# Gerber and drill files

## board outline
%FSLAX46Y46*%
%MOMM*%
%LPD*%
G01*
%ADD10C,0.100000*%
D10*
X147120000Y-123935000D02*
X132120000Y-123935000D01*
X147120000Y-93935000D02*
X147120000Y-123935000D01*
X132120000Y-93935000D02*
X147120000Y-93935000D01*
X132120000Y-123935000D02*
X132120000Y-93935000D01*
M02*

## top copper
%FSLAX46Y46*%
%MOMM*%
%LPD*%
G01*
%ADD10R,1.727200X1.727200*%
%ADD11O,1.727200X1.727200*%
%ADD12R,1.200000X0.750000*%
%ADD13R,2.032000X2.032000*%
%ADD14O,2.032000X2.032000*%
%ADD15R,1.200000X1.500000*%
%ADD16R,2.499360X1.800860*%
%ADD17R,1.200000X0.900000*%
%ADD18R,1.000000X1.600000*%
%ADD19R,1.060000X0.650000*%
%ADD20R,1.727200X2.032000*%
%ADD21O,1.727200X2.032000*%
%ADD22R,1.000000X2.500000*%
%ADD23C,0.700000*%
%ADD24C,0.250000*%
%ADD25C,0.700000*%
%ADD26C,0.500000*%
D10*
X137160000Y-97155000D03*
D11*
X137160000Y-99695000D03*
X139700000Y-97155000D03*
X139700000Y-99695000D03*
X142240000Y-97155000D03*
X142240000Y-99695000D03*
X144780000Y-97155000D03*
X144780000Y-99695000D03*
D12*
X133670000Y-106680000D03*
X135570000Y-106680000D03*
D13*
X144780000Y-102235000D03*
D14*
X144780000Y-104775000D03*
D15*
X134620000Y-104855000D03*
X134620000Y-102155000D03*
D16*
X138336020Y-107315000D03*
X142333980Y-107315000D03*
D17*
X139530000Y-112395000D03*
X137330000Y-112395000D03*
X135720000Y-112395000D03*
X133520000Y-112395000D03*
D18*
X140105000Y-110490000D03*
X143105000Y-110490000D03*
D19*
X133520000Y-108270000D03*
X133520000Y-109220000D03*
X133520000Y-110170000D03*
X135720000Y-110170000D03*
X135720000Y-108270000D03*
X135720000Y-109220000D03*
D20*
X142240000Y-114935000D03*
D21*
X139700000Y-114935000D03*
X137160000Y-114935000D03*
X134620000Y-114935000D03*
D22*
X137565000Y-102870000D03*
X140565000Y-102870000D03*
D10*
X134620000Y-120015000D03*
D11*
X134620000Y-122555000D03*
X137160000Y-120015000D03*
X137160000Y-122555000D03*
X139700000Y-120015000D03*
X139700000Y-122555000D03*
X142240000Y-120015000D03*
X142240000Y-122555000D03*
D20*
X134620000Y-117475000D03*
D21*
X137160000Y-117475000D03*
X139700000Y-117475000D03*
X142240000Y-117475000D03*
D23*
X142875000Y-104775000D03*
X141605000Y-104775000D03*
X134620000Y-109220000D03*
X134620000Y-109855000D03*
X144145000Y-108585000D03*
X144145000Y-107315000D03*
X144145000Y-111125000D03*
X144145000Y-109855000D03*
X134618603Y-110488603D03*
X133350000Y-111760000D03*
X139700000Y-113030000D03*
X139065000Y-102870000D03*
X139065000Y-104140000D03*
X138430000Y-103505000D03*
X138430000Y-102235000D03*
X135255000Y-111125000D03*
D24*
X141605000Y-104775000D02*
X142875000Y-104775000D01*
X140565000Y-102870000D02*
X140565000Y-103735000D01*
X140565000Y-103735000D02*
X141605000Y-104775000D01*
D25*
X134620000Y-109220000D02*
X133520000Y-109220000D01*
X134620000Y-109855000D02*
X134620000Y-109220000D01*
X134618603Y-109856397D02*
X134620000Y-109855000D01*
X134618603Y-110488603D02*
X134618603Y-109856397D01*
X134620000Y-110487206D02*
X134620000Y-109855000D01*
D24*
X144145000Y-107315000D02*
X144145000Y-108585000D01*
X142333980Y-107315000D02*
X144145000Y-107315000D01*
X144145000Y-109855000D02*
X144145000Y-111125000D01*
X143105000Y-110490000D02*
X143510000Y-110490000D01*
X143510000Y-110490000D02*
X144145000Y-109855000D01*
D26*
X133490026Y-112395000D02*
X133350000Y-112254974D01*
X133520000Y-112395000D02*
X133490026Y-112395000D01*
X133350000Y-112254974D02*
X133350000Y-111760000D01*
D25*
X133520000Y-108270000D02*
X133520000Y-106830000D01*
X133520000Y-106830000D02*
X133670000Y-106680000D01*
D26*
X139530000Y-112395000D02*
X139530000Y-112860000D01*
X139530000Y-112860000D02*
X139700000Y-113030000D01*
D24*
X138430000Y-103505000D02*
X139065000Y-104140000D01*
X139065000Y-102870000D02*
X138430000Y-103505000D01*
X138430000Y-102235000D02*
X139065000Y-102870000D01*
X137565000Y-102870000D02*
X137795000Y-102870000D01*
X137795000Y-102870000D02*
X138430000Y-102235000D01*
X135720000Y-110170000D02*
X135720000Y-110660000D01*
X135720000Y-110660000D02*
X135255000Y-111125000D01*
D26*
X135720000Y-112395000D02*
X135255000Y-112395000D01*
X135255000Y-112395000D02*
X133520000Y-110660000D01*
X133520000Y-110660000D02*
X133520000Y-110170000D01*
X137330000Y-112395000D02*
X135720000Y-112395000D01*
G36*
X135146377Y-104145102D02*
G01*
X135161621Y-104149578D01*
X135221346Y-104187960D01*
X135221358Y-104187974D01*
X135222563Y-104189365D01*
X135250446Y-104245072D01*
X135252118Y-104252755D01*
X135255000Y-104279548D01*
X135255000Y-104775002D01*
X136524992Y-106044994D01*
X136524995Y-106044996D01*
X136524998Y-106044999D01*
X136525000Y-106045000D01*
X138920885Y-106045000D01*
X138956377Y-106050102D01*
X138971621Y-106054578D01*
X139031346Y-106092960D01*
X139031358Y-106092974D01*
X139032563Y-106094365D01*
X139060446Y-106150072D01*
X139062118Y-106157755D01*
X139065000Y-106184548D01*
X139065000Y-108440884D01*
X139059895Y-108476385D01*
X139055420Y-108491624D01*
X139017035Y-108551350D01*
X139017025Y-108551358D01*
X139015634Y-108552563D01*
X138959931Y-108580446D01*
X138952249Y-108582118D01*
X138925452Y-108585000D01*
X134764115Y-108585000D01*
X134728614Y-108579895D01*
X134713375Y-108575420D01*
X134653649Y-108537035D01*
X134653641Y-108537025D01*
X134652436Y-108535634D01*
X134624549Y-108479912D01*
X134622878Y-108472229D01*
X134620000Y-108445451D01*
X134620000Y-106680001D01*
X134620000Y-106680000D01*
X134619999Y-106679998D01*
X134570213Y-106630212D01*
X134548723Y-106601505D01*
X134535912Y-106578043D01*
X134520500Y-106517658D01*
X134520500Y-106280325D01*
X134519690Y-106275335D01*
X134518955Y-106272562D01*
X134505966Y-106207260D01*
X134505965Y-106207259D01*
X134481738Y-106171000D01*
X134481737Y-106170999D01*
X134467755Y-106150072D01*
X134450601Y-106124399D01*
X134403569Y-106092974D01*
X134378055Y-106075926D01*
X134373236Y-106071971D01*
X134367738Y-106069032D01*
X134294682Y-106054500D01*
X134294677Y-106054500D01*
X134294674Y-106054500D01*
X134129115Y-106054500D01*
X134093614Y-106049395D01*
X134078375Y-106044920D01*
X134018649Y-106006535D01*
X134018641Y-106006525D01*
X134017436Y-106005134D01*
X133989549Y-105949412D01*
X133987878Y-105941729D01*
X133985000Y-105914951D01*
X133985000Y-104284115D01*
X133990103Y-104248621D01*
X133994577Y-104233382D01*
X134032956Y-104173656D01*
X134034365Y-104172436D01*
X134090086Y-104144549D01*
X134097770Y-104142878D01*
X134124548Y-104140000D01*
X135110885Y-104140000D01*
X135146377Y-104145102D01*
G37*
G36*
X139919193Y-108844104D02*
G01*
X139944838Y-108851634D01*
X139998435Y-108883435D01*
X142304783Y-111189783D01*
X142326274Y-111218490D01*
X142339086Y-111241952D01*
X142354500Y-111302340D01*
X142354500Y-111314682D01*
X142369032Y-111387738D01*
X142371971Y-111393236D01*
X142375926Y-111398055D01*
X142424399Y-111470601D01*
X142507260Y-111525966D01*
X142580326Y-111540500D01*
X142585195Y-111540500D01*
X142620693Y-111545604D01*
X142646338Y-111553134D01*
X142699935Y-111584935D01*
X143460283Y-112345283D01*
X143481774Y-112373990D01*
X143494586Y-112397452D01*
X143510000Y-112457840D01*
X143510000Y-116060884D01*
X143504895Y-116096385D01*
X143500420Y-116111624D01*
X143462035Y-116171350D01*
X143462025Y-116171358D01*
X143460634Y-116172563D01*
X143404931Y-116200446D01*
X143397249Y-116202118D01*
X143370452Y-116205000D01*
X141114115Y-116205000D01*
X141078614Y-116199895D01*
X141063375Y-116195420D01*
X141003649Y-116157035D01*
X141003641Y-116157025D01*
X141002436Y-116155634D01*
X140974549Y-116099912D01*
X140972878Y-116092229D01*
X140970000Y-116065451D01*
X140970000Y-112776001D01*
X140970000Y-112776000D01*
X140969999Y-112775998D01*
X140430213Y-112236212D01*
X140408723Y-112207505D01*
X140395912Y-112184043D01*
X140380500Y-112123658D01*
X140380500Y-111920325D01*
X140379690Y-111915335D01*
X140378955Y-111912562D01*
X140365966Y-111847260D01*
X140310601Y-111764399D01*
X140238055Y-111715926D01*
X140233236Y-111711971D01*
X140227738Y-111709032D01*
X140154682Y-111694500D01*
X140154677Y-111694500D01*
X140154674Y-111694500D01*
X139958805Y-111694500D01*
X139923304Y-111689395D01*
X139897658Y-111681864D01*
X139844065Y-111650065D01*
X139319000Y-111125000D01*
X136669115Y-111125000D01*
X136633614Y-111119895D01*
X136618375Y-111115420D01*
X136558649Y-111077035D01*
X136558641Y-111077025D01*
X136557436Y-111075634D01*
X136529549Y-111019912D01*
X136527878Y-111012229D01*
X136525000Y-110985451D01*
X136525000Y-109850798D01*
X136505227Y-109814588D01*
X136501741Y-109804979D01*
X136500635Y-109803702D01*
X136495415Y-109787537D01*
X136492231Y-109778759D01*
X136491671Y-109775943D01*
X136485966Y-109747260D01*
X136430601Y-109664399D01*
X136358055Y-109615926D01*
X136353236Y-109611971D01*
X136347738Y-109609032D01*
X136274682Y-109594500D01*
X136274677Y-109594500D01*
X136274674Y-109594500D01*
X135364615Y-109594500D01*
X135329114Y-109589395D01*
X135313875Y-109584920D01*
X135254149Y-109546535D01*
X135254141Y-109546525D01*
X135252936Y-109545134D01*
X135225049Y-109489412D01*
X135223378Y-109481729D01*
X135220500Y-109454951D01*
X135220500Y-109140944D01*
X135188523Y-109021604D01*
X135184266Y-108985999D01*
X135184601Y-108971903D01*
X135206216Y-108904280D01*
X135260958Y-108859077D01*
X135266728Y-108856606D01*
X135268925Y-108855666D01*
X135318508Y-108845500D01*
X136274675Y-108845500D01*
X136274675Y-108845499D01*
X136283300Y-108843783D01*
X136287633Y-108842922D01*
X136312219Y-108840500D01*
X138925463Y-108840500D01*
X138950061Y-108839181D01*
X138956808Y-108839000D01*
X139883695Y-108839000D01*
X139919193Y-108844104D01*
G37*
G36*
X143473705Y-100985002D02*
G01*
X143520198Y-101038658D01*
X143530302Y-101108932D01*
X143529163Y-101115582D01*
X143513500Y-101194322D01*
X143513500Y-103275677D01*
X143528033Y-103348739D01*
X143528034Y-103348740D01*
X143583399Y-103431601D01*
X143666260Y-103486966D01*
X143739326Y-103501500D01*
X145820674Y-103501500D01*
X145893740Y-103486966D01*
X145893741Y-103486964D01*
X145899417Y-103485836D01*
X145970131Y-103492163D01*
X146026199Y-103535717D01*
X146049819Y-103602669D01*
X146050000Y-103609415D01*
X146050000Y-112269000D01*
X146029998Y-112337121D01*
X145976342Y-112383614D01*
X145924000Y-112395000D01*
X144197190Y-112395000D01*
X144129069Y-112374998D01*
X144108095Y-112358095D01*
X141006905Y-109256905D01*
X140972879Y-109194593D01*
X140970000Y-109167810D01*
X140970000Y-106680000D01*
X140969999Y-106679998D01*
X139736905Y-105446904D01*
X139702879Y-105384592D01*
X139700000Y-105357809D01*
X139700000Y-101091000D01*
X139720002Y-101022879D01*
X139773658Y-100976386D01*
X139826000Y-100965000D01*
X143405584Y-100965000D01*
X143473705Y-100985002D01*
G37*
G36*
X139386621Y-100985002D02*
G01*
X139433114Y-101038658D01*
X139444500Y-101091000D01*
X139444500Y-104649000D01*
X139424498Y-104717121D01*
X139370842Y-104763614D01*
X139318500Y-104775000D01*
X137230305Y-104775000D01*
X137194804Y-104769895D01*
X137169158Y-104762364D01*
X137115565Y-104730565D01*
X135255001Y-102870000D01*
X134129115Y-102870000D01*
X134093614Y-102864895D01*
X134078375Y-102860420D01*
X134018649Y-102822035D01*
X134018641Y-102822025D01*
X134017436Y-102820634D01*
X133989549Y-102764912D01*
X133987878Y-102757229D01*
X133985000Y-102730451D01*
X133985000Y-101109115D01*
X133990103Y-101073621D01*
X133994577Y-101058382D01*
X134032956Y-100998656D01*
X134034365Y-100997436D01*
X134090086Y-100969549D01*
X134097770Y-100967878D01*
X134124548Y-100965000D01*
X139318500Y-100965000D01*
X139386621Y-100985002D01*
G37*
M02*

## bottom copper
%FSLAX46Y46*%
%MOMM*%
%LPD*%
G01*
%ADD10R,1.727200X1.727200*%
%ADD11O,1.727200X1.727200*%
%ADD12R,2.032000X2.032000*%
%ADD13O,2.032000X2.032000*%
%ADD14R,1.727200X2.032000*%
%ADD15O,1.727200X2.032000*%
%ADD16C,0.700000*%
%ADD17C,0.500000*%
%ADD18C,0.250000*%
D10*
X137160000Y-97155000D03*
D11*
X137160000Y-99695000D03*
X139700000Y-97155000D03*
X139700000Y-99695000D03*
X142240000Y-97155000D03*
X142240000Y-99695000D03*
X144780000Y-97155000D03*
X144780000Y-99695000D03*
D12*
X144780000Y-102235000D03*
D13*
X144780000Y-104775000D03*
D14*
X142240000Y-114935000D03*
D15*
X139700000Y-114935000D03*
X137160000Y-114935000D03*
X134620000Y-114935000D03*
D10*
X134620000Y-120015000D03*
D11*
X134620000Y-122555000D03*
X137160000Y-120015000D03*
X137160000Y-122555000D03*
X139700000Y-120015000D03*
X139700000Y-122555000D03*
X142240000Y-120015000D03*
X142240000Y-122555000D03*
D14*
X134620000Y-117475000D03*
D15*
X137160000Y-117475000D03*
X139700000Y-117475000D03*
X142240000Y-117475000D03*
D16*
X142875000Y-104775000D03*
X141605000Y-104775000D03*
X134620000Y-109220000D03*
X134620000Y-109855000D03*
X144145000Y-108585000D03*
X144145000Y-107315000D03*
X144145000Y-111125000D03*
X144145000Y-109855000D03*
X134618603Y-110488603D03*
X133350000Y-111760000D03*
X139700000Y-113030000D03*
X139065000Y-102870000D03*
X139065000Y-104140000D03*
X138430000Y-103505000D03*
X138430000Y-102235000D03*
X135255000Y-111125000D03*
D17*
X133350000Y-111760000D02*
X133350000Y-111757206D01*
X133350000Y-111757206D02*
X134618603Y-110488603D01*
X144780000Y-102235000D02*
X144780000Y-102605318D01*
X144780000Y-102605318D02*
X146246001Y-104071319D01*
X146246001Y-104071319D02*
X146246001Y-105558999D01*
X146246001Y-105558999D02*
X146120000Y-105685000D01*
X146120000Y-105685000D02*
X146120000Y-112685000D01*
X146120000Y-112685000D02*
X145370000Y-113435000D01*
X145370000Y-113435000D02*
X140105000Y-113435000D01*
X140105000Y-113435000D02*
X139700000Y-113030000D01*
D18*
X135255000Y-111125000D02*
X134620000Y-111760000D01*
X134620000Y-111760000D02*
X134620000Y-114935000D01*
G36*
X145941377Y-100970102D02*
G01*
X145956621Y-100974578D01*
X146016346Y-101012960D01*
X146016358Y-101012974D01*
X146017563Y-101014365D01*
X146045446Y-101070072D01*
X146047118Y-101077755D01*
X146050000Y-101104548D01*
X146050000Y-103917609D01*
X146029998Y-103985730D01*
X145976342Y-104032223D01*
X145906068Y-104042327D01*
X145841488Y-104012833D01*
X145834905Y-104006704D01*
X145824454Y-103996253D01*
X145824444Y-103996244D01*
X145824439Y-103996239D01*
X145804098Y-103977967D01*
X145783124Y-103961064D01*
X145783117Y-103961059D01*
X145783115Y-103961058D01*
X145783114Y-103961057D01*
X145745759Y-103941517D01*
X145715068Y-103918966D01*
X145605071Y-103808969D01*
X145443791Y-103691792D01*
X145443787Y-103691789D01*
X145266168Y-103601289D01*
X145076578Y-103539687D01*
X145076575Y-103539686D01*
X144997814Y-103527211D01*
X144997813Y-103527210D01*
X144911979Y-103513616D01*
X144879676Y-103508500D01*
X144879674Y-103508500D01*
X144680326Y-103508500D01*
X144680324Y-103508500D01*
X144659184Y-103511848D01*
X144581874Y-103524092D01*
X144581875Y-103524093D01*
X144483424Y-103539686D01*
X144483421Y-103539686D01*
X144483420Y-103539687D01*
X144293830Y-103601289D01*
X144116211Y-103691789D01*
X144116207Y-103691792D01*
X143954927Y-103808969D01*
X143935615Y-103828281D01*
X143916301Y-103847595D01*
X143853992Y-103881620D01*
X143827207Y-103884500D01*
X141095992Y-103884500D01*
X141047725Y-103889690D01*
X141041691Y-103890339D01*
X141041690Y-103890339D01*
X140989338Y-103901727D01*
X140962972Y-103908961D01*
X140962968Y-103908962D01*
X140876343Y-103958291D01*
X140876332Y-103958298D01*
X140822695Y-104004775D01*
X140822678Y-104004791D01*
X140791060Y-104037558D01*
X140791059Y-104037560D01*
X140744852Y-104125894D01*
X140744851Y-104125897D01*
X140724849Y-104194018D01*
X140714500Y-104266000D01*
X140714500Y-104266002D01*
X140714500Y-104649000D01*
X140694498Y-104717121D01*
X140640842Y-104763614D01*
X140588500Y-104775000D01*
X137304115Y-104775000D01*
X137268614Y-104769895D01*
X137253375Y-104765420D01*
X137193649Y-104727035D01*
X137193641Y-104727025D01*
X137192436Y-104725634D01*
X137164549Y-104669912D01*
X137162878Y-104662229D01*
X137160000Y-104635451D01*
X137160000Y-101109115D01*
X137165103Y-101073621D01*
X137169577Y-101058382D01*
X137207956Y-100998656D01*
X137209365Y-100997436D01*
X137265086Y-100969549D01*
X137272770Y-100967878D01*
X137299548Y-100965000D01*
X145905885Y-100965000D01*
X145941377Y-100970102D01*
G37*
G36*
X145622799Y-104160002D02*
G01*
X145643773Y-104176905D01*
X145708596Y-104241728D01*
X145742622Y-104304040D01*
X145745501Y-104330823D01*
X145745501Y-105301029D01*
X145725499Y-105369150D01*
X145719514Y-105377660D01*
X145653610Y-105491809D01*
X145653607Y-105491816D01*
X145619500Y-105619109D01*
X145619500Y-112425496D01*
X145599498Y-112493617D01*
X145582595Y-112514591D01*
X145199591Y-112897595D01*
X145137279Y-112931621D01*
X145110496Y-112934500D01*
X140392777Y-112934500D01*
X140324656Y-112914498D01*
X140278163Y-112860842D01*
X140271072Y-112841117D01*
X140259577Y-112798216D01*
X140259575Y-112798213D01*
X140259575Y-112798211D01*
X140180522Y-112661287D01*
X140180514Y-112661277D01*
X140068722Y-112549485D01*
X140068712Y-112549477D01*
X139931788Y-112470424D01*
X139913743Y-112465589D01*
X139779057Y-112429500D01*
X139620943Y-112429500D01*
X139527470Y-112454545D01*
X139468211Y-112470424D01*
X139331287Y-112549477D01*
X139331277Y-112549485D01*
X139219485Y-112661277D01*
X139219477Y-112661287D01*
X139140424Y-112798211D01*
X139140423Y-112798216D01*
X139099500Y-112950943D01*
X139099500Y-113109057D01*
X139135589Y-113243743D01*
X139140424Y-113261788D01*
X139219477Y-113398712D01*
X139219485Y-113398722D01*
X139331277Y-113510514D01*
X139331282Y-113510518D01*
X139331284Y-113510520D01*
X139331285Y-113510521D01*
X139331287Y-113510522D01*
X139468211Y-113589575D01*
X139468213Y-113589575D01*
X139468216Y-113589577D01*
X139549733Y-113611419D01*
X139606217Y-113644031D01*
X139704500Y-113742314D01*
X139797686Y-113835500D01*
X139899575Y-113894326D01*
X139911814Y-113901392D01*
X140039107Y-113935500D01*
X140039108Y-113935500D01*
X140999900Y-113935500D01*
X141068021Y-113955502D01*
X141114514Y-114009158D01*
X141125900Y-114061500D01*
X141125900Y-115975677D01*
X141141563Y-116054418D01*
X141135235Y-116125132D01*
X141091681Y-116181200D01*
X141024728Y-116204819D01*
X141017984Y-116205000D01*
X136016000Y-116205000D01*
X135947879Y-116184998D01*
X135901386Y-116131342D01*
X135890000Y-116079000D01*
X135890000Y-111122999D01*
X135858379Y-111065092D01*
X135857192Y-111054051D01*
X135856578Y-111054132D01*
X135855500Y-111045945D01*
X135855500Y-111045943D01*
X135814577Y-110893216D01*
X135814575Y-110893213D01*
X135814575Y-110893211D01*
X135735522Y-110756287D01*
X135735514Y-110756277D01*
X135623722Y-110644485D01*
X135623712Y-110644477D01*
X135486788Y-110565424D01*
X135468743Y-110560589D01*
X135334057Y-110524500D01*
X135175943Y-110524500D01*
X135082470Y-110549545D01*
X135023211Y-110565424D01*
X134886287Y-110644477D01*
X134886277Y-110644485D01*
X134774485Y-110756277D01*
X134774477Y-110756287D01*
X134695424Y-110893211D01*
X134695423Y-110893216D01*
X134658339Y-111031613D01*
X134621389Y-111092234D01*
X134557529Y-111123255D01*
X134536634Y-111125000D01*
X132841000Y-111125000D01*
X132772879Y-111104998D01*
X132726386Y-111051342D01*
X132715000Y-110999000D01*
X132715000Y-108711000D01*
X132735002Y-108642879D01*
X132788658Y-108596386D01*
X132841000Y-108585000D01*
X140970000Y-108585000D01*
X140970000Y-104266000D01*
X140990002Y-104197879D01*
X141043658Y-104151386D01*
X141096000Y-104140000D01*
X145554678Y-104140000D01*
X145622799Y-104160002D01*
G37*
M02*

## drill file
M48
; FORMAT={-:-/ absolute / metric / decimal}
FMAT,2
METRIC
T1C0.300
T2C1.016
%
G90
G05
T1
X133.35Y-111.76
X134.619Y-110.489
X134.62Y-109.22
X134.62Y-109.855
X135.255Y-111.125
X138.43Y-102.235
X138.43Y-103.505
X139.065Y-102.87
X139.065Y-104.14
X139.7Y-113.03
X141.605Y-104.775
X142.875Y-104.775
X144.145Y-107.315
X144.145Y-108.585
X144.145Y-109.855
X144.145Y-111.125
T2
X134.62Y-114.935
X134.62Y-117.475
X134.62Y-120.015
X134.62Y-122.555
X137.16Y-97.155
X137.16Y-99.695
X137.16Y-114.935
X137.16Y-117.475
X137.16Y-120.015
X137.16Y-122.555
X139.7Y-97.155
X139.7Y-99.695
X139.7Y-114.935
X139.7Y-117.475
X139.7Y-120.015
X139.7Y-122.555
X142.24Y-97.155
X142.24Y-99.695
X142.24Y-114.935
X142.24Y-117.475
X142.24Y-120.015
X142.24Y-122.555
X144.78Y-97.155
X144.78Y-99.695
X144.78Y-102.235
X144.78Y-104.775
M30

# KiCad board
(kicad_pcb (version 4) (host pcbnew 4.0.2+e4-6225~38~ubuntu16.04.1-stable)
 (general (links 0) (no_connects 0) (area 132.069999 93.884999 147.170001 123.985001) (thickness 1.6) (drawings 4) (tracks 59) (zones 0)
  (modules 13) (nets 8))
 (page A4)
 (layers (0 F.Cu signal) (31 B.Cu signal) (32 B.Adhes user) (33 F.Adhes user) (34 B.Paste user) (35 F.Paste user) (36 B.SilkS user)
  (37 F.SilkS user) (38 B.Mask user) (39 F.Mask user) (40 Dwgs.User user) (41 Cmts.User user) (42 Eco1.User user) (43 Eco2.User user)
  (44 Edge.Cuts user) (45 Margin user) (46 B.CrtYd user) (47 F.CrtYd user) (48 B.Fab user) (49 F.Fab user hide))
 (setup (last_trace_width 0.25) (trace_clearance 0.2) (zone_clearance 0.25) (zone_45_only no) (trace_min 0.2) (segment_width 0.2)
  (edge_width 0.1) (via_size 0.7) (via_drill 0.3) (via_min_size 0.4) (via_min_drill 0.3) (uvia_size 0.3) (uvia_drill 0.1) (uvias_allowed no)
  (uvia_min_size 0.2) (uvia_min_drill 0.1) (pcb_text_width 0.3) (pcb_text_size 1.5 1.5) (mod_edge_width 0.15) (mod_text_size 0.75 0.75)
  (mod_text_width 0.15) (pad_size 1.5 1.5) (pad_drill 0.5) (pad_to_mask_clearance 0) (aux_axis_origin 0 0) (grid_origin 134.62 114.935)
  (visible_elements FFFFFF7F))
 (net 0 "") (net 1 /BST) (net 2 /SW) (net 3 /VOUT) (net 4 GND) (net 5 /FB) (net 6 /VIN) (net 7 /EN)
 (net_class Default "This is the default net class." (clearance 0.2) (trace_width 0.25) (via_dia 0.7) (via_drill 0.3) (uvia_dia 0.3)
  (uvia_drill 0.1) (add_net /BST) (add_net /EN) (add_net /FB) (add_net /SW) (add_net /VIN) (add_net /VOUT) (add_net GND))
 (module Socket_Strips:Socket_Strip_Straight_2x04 (layer F.Cu) (at 137.16 97.155)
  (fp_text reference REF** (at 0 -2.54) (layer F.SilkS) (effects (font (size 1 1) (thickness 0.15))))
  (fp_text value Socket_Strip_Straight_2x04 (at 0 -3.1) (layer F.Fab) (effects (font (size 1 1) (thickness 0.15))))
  (pad 1 thru_hole rect (at 0 0) (size 1.7272 1.7272) (drill 1.016) (layers *.Cu *.Mask F.SilkS))
  (pad 2 thru_hole oval (at 0 2.54) (size 1.7272 1.7272) (drill 1.016) (layers *.Cu *.Mask F.SilkS))
  (pad 3 thru_hole oval (at 2.54 0) (size 1.7272 1.7272) (drill 1.016) (layers *.Cu *.Mask F.SilkS))
  (pad 4 thru_hole oval (at 2.54 2.54) (size 1.7272 1.7272) (drill 1.016) (layers *.Cu *.Mask F.SilkS))
  (pad 5 thru_hole oval (at 5.08 0) (size 1.7272 1.7272) (drill 1.016) (layers *.Cu *.Mask F.SilkS))
  (pad 6 thru_hole oval (at 5.08 2.54) (size 1.7272 1.7272) (drill 1.016) (layers *.Cu *.Mask F.SilkS))
  (pad 7 thru_hole oval (at 7.62 0) (size 1.7272 1.7272) (drill 1.016) (layers *.Cu *.Mask F.SilkS))
  (pad 8 thru_hole oval (at 7.62 2.54) (size 1.7272 1.7272) (drill 1.016) (layers *.Cu *.Mask F.SilkS)))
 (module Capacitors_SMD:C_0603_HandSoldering (layer F.Cu) (at 134.62 106.68)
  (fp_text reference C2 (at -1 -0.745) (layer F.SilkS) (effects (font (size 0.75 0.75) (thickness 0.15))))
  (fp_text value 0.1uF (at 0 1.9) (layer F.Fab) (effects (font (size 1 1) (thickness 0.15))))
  (pad 1 smd rect (at -0.95 0) (size 1.2 0.75) (layers F.Cu F.Paste F.Mask) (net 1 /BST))
  (pad 2 smd rect (at 0.95 0) (size 1.2 0.75) (layers F.Cu F.Paste F.Mask) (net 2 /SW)))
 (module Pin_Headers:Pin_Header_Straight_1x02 (layer F.Cu) (at 144.78 102.235)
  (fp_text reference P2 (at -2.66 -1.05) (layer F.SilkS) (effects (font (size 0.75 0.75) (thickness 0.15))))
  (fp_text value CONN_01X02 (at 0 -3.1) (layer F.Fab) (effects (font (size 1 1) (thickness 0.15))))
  (pad 1 thru_hole rect (at 0 0) (size 2.032 2.032) (drill 1.016) (layers *.Cu *.Mask F.SilkS) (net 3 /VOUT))
  (pad 2 thru_hole oval (at 0 2.54) (size 2.032 2.032) (drill 1.016) (layers *.Cu *.Mask F.SilkS) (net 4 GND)))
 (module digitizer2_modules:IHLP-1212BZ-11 (layer F.Cu) (at 134.62 103.505 90)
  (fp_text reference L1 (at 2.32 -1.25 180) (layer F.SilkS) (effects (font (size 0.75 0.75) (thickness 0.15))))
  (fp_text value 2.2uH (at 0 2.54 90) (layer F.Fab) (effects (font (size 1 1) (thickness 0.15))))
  (pad 1 smd rect (at -1.35 0 90) (size 1.5 1.2) (layers F.Cu F.Paste F.Mask) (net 2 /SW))
  (pad 2 smd rect (at 1.35 0 90) (size 1.5 1.2) (layers F.Cu F.Paste F.Mask) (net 3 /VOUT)))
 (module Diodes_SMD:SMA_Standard (layer F.Cu) (at 140.335 107.315)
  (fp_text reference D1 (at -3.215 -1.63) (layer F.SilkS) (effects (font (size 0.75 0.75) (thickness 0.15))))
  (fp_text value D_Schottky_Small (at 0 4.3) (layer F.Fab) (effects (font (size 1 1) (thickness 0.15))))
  (pad 1 smd rect (at -1.99898 0) (size 2.49936 1.80086) (layers F.Cu F.Paste F.Mask) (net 2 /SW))
  (pad 2 smd rect (at 1.99898 0) (size 2.49936 1.80086) (layers F.Cu F.Paste F.Mask) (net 4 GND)))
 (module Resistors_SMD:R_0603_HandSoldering (layer F.Cu) (at 138.43 112.395 180)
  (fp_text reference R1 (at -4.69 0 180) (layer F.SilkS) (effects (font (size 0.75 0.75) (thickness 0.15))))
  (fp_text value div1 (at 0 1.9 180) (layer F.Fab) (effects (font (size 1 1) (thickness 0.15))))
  (pad 1 smd rect (at -1.1 0 180) (size 1.2 0.9) (layers F.Cu F.Paste F.Mask) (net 3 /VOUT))
  (pad 2 smd rect (at 1.1 0 180) (size 1.2 0.9) (layers F.Cu F.Paste F.Mask) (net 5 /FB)))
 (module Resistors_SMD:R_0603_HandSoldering (layer F.Cu) (at 134.62 112.395 180)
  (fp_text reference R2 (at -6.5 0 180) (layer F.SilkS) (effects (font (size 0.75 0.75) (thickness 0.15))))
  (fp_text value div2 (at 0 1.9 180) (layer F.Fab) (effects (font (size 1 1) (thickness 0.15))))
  (pad 1 smd rect (at -1.1 0 180) (size 1.2 0.9) (layers F.Cu F.Paste F.Mask) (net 5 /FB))
  (pad 2 smd rect (at 1.1 0 180) (size 1.2 0.9) (layers F.Cu F.Paste F.Mask) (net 4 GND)))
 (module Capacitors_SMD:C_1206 (layer F.Cu) (at 141.605 110.49)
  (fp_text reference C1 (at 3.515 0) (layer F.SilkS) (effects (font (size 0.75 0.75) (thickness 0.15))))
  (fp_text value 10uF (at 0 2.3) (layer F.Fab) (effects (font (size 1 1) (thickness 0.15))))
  (pad 1 smd rect (at -1.5 0) (size 1 1.6) (layers F.Cu F.Paste F.Mask) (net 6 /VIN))
  (pad 2 smd rect (at 1.5 0) (size 1 1.6) (layers F.Cu F.Paste F.Mask) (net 4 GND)))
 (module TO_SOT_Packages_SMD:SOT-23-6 (layer F.Cu) (at 134.62 109.22)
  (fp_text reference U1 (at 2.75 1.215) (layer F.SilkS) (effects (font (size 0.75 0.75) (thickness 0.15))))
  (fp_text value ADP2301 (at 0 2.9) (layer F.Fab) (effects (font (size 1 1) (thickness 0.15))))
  (pad 1 smd rect (at -1.1 -0.95) (size 1.06 0.65) (layers F.Cu F.Paste F.Mask) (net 1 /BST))
  (pad 2 smd rect (at -1.1 0) (size 1.06 0.65) (layers F.Cu F.Paste F.Mask) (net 4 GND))
  (pad 3 smd rect (at -1.1 0.95) (size 1.06 0.65) (layers F.Cu F.Paste F.Mask) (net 5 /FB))
  (pad 4 smd rect (at 1.1 0.95) (size 1.06 0.65) (layers F.Cu F.Paste F.Mask) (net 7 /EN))
  (pad 6 smd rect (at 1.1 -0.95) (size 1.06 0.65) (layers F.Cu F.Paste F.Mask) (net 2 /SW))
  (pad 5 smd rect (at 1.1 0) (size 1.06 0.65) (layers F.Cu F.Paste F.Mask) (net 6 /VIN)))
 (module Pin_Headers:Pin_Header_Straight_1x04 (layer F.Cu) (at 142.24 114.935 270)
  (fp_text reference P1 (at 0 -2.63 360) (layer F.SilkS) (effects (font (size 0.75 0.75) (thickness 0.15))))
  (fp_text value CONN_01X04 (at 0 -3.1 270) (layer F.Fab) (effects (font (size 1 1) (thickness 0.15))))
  (pad 1 thru_hole rect (at 0 0 270) (size 2.032 1.7272) (drill 1.016) (layers *.Cu *.Mask F.SilkS) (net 6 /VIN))
  (pad 2 thru_hole oval (at 0 2.54 270) (size 2.032 1.7272) (drill 1.016) (layers *.Cu *.Mask F.SilkS) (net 4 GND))
  (pad 3 thru_hole oval (at 0 5.08 270) (size 2.032 1.7272) (drill 1.016) (layers *.Cu *.Mask F.SilkS) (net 4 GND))
  (pad 4 thru_hole oval (at 0 7.62 270) (size 2.032 1.7272) (drill 1.016) (layers *.Cu *.Mask F.SilkS) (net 7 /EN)))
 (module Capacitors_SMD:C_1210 (layer F.Cu) (at 139.065 102.87)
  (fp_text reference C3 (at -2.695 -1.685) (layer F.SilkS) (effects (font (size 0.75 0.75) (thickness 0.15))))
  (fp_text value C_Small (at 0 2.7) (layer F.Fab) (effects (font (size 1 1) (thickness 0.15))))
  (pad 1 smd rect (at -1.5 0) (size 1 2.5) (layers F.Cu F.Paste F.Mask) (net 3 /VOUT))
  (pad 2 smd rect (at 1.5 0) (size 1 2.5) (layers F.Cu F.Paste F.Mask) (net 4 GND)))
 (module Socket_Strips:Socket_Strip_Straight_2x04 (layer F.Cu) (at 134.62 120.015)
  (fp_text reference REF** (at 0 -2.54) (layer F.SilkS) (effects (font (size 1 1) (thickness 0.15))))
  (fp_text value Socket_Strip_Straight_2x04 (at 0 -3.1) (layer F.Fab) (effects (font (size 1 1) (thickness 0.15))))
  (pad 1 thru_hole rect (at 0 0) (size 1.7272 1.7272) (drill 1.016) (layers *.Cu *.Mask F.SilkS))
  (pad 2 thru_hole oval (at 0 2.54) (size 1.7272 1.7272) (drill 1.016) (layers *.Cu *.Mask F.SilkS))
  (pad 3 thru_hole oval (at 2.54 0) (size 1.7272 1.7272) (drill 1.016) (layers *.Cu *.Mask F.SilkS))
  (pad 4 thru_hole oval (at 2.54 2.54) (size 1.7272 1.7272) (drill 1.016) (layers *.Cu *.Mask F.SilkS))
  (pad 5 thru_hole oval (at 5.08 0) (size 1.7272 1.7272) (drill 1.016) (layers *.Cu *.Mask F.SilkS))
  (pad 6 thru_hole oval (at 5.08 2.54) (size 1.7272 1.7272) (drill 1.016) (layers *.Cu *.Mask F.SilkS))
  (pad 7 thru_hole oval (at 7.62 0) (size 1.7272 1.7272) (drill 1.016) (layers *.Cu *.Mask F.SilkS))
  (pad 8 thru_hole oval (at 7.62 2.54) (size 1.7272 1.7272) (drill 1.016) (layers *.Cu *.Mask F.SilkS)))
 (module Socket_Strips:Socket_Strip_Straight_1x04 (layer F.Cu) (at 134.62 117.475)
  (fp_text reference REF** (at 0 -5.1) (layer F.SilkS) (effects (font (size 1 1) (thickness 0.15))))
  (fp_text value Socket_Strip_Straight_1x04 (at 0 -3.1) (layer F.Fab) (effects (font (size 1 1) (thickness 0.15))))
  (pad 1 thru_hole rect (at 0 0) (size 1.7272 2.032) (drill 1.016) (layers *.Cu *.Mask F.SilkS))
  (pad 2 thru_hole oval (at 2.54 0) (size 1.7272 2.032) (drill 1.016) (layers *.Cu *.Mask F.SilkS))
  (pad 3 thru_hole oval (at 5.08 0) (size 1.7272 2.032) (drill 1.016) (layers *.Cu *.Mask F.SilkS))
  (pad 4 thru_hole oval (at 7.62 0) (size 1.7272 2.032) (drill 1.016) (layers *.Cu *.Mask F.SilkS)))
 (gr_line (start 147.12 123.935) (end 132.12 123.935) (layer Edge.Cuts) (width 0.1))
 (gr_line (start 147.12 93.935) (end 147.12 123.935) (layer Edge.Cuts) (width 0.1))
 (gr_line (start 132.12 93.935) (end 147.12 93.935) (layer Edge.Cuts) (width 0.1))
 (gr_line (start 132.12 123.935) (end 132.12 93.935) (layer Edge.Cuts) (width 0.1))
 (segment (start 141.605 104.775) (end 142.875 104.775) (width 0.25) (layer F.Cu) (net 4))
 (via (at 142.875 104.775) (size 0.7) (drill 0.3) (layers F.Cu B.Cu) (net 4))
 (segment (start 140.565 102.87) (end 140.565 103.735) (width 0.25) (layer F.Cu) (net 4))
 (segment (start 140.565 103.735) (end 141.605 104.775) (width 0.25) (layer F.Cu) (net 4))
 (via (at 141.605 104.775) (size 0.7) (drill 0.3) (layers F.Cu B.Cu) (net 4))
 (segment (start 134.62 109.22) (end 133.52 109.22) (width 0.7) (layer F.Cu) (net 4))
 (segment (start 134.62 109.855) (end 134.62 109.22) (width 0.7) (layer F.Cu) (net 4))
 (via (at 134.62 109.22) (size 0.7) (drill 0.3) (layers F.Cu B.Cu) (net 4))
 (segment (start 134.618603 109.856397) (end 134.62 109.855) (width 0.7) (layer F.Cu) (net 4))
 (segment (start 134.618603 110.488603) (end 134.618603 109.856397) (width 0.7) (layer F.Cu) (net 4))
 (segment (start 134.62 110.487206) (end 134.62 109.855) (width 0.7) (layer F.Cu) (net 4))
 (via (at 134.62 109.855) (size 0.7) (drill 0.3) (layers F.Cu B.Cu) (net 4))
 (segment (start 144.145 107.315) (end 144.145 108.585) (width 0.25) (layer F.Cu) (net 4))
 (via (at 144.145 108.585) (size 0.7) (drill 0.3) (layers F.Cu B.Cu) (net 4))
 (segment (start 142.33398 107.315) (end 144.145 107.315) (width 0.25) (layer F.Cu) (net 4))
 (via (at 144.145 107.315) (size 0.7) (drill 0.3) (layers F.Cu B.Cu) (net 4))
 (segment (start 144.145 109.855) (end 144.145 111.125) (width 0.25) (layer F.Cu) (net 4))
 (via (at 144.145 111.125) (size 0.7) (drill 0.3) (layers F.Cu B.Cu) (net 4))
 (segment (start 143.105 110.49) (end 143.51 110.49) (width 0.25) (layer F.Cu) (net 4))
 (segment (start 143.51 110.49) (end 144.145 109.855) (width 0.25) (layer F.Cu) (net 4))
 (via (at 144.145 109.855) (size 0.7) (drill 0.3) (layers F.Cu B.Cu) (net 4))
 (segment (start 133.35 111.76) (end 133.35 111.757206) (width 0.5) (layer B.Cu) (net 4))
 (segment (start 133.35 111.757206) (end 134.618603 110.488603) (width 0.5) (layer B.Cu) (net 4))
 (via (at 134.618603 110.488603) (size 0.7) (drill 0.3) (layers F.Cu B.Cu) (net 4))
 (segment (start 133.490026 112.395) (end 133.35 112.254974) (width 0.5) (layer F.Cu) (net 4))
 (segment (start 133.52 112.395) (end 133.490026 112.395) (width 0.5) (layer F.Cu) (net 4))
 (segment (start 133.35 112.254974) (end 133.35 111.76) (width 0.5) (layer F.Cu) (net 4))
 (via (at 133.35 111.76) (size 0.7) (drill 0.3) (layers F.Cu B.Cu) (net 4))
 (segment (start 133.52 108.27) (end 133.52 106.83) (width 0.7) (layer F.Cu) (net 1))
 (segment (start 133.52 106.83) (end 133.67 106.68) (width 0.7) (layer F.Cu) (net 1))
 (segment (start 144.78 102.235) (end 144.78 102.605318) (width 0.5) (layer B.Cu) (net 3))
 (segment (start 144.78 102.605318) (end 146.246001 104.071319) (width 0.5) (layer B.Cu) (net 3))
 (segment (start 146.246001 104.071319) (end 146.246001 105.558999) (width 0.5) (layer B.Cu) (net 3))
 (segment (start 146.246001 105.558999) (end 146.12 105.685) (width 0.5) (layer B.Cu) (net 3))
 (segment (start 146.12 105.685) (end 146.12 112.685) (width 0.5) (layer B.Cu) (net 3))
 (segment (start 146.12 112.685) (end 145.37 113.435) (width 0.5) (layer B.Cu) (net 3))
 (segment (start 145.37 113.435) (end 140.105 113.435) (width 0.5) (layer B.Cu) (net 3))
 (segment (start 140.105 113.435) (end 139.7 113.03) (width 0.5) (layer B.Cu) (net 3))
 (segment (start 139.53 112.395) (end 139.53 112.86) (width 0.5) (layer F.Cu) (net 3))
 (segment (start 139.53 112.86) (end 139.7 113.03) (width 0.5) (layer F.Cu) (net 3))
 (via (at 139.7 113.03) (size 0.7) (drill 0.3) (layers F.Cu B.Cu) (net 3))
 (via (at 139.065 102.87) (size 0.7) (drill 0.3) (layers F.Cu B.Cu) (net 3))
 (segment (start 138.43 103.505) (end 139.065 104.14) (width 0.25) (layer F.Cu) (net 3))
 (via (at 139.065 104.14) (size 0.7) (drill 0.3) (layers F.Cu B.Cu) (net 3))
 (segment (start 139.065 102.87) (end 138.43 103.505) (width 0.25) (layer F.Cu) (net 3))
 (via (at 138.43 103.505) (size 0.7) (drill 0.3) (layers F.Cu B.Cu) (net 3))
 (segment (start 138.43 102.235) (end 139.065 102.87) (width 0.25) (layer F.Cu) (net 3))
 (segment (start 137.565 102.87) (end 137.795 102.87) (width 0.25) (layer F.Cu) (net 3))
 (segment (start 137.795 102.87) (end 138.43 102.235) (width 0.25) (layer F.Cu) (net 3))
 (via (at 138.43 102.235) (size 0.7) (drill 0.3) (layers F.Cu B.Cu) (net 3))
 (segment (start 135.255 111.125) (end 134.62 111.76) (width 0.25) (layer B.Cu) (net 7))
 (segment (start 134.62 111.76) (end 134.62 114.935) (width 0.25) (layer B.Cu) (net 7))
 (segment (start 135.72 110.17) (end 135.72 110.66) (width 0.25) (layer F.Cu) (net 7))
 (segment (start 135.72 110.66) (end 135.255 111.125) (width 0.25) (layer F.Cu) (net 7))
 (via (at 135.255 111.125) (size 0.7) (drill 0.3) (layers F.Cu B.Cu) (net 7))
 (segment (start 135.72 112.395) (end 135.255 112.395) (width 0.5) (layer F.Cu) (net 5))
 (segment (start 135.255 112.395) (end 133.52 110.66) (width 0.5) (layer F.Cu) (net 5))
 (segment (start 133.52 110.66) (end 133.52 110.17) (width 0.5) (layer F.Cu) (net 5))
 (segment (start 137.33 112.395) (end 135.72 112.395) (width 0.5) (layer F.Cu) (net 5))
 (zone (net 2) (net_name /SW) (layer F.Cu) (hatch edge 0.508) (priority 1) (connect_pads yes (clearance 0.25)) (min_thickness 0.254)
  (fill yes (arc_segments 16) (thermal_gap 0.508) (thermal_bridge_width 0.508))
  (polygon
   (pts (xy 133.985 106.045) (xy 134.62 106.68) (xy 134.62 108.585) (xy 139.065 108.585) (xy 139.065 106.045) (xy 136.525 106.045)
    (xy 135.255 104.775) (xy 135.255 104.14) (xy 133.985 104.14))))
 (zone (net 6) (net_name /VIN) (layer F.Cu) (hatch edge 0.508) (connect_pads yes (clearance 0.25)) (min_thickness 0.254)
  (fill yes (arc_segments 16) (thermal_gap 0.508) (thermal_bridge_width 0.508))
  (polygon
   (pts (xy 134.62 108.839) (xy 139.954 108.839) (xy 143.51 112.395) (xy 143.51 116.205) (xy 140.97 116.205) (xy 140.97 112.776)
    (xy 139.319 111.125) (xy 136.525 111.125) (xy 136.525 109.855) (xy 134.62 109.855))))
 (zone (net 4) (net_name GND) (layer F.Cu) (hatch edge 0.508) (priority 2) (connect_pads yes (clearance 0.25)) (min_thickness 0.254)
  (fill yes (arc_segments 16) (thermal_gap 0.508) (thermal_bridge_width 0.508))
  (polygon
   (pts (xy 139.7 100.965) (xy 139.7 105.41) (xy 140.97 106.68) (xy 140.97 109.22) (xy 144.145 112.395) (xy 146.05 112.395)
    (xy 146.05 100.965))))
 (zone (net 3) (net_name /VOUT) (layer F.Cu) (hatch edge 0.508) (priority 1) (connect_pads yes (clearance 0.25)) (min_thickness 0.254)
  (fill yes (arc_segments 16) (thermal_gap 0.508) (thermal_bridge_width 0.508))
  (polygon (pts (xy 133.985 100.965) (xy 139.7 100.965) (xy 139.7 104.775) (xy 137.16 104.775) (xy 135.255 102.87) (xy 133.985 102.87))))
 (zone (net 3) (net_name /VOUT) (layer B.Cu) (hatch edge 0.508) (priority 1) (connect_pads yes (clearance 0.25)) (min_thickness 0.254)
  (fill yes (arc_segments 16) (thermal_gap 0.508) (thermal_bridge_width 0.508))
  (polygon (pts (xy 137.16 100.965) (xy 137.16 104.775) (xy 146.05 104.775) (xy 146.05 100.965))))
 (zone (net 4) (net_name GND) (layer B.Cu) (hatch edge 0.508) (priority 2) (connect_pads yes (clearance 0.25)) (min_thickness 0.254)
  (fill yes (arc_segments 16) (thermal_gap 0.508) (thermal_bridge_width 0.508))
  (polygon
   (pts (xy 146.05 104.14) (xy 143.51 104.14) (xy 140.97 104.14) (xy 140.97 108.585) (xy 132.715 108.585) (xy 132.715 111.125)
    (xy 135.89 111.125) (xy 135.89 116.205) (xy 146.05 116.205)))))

